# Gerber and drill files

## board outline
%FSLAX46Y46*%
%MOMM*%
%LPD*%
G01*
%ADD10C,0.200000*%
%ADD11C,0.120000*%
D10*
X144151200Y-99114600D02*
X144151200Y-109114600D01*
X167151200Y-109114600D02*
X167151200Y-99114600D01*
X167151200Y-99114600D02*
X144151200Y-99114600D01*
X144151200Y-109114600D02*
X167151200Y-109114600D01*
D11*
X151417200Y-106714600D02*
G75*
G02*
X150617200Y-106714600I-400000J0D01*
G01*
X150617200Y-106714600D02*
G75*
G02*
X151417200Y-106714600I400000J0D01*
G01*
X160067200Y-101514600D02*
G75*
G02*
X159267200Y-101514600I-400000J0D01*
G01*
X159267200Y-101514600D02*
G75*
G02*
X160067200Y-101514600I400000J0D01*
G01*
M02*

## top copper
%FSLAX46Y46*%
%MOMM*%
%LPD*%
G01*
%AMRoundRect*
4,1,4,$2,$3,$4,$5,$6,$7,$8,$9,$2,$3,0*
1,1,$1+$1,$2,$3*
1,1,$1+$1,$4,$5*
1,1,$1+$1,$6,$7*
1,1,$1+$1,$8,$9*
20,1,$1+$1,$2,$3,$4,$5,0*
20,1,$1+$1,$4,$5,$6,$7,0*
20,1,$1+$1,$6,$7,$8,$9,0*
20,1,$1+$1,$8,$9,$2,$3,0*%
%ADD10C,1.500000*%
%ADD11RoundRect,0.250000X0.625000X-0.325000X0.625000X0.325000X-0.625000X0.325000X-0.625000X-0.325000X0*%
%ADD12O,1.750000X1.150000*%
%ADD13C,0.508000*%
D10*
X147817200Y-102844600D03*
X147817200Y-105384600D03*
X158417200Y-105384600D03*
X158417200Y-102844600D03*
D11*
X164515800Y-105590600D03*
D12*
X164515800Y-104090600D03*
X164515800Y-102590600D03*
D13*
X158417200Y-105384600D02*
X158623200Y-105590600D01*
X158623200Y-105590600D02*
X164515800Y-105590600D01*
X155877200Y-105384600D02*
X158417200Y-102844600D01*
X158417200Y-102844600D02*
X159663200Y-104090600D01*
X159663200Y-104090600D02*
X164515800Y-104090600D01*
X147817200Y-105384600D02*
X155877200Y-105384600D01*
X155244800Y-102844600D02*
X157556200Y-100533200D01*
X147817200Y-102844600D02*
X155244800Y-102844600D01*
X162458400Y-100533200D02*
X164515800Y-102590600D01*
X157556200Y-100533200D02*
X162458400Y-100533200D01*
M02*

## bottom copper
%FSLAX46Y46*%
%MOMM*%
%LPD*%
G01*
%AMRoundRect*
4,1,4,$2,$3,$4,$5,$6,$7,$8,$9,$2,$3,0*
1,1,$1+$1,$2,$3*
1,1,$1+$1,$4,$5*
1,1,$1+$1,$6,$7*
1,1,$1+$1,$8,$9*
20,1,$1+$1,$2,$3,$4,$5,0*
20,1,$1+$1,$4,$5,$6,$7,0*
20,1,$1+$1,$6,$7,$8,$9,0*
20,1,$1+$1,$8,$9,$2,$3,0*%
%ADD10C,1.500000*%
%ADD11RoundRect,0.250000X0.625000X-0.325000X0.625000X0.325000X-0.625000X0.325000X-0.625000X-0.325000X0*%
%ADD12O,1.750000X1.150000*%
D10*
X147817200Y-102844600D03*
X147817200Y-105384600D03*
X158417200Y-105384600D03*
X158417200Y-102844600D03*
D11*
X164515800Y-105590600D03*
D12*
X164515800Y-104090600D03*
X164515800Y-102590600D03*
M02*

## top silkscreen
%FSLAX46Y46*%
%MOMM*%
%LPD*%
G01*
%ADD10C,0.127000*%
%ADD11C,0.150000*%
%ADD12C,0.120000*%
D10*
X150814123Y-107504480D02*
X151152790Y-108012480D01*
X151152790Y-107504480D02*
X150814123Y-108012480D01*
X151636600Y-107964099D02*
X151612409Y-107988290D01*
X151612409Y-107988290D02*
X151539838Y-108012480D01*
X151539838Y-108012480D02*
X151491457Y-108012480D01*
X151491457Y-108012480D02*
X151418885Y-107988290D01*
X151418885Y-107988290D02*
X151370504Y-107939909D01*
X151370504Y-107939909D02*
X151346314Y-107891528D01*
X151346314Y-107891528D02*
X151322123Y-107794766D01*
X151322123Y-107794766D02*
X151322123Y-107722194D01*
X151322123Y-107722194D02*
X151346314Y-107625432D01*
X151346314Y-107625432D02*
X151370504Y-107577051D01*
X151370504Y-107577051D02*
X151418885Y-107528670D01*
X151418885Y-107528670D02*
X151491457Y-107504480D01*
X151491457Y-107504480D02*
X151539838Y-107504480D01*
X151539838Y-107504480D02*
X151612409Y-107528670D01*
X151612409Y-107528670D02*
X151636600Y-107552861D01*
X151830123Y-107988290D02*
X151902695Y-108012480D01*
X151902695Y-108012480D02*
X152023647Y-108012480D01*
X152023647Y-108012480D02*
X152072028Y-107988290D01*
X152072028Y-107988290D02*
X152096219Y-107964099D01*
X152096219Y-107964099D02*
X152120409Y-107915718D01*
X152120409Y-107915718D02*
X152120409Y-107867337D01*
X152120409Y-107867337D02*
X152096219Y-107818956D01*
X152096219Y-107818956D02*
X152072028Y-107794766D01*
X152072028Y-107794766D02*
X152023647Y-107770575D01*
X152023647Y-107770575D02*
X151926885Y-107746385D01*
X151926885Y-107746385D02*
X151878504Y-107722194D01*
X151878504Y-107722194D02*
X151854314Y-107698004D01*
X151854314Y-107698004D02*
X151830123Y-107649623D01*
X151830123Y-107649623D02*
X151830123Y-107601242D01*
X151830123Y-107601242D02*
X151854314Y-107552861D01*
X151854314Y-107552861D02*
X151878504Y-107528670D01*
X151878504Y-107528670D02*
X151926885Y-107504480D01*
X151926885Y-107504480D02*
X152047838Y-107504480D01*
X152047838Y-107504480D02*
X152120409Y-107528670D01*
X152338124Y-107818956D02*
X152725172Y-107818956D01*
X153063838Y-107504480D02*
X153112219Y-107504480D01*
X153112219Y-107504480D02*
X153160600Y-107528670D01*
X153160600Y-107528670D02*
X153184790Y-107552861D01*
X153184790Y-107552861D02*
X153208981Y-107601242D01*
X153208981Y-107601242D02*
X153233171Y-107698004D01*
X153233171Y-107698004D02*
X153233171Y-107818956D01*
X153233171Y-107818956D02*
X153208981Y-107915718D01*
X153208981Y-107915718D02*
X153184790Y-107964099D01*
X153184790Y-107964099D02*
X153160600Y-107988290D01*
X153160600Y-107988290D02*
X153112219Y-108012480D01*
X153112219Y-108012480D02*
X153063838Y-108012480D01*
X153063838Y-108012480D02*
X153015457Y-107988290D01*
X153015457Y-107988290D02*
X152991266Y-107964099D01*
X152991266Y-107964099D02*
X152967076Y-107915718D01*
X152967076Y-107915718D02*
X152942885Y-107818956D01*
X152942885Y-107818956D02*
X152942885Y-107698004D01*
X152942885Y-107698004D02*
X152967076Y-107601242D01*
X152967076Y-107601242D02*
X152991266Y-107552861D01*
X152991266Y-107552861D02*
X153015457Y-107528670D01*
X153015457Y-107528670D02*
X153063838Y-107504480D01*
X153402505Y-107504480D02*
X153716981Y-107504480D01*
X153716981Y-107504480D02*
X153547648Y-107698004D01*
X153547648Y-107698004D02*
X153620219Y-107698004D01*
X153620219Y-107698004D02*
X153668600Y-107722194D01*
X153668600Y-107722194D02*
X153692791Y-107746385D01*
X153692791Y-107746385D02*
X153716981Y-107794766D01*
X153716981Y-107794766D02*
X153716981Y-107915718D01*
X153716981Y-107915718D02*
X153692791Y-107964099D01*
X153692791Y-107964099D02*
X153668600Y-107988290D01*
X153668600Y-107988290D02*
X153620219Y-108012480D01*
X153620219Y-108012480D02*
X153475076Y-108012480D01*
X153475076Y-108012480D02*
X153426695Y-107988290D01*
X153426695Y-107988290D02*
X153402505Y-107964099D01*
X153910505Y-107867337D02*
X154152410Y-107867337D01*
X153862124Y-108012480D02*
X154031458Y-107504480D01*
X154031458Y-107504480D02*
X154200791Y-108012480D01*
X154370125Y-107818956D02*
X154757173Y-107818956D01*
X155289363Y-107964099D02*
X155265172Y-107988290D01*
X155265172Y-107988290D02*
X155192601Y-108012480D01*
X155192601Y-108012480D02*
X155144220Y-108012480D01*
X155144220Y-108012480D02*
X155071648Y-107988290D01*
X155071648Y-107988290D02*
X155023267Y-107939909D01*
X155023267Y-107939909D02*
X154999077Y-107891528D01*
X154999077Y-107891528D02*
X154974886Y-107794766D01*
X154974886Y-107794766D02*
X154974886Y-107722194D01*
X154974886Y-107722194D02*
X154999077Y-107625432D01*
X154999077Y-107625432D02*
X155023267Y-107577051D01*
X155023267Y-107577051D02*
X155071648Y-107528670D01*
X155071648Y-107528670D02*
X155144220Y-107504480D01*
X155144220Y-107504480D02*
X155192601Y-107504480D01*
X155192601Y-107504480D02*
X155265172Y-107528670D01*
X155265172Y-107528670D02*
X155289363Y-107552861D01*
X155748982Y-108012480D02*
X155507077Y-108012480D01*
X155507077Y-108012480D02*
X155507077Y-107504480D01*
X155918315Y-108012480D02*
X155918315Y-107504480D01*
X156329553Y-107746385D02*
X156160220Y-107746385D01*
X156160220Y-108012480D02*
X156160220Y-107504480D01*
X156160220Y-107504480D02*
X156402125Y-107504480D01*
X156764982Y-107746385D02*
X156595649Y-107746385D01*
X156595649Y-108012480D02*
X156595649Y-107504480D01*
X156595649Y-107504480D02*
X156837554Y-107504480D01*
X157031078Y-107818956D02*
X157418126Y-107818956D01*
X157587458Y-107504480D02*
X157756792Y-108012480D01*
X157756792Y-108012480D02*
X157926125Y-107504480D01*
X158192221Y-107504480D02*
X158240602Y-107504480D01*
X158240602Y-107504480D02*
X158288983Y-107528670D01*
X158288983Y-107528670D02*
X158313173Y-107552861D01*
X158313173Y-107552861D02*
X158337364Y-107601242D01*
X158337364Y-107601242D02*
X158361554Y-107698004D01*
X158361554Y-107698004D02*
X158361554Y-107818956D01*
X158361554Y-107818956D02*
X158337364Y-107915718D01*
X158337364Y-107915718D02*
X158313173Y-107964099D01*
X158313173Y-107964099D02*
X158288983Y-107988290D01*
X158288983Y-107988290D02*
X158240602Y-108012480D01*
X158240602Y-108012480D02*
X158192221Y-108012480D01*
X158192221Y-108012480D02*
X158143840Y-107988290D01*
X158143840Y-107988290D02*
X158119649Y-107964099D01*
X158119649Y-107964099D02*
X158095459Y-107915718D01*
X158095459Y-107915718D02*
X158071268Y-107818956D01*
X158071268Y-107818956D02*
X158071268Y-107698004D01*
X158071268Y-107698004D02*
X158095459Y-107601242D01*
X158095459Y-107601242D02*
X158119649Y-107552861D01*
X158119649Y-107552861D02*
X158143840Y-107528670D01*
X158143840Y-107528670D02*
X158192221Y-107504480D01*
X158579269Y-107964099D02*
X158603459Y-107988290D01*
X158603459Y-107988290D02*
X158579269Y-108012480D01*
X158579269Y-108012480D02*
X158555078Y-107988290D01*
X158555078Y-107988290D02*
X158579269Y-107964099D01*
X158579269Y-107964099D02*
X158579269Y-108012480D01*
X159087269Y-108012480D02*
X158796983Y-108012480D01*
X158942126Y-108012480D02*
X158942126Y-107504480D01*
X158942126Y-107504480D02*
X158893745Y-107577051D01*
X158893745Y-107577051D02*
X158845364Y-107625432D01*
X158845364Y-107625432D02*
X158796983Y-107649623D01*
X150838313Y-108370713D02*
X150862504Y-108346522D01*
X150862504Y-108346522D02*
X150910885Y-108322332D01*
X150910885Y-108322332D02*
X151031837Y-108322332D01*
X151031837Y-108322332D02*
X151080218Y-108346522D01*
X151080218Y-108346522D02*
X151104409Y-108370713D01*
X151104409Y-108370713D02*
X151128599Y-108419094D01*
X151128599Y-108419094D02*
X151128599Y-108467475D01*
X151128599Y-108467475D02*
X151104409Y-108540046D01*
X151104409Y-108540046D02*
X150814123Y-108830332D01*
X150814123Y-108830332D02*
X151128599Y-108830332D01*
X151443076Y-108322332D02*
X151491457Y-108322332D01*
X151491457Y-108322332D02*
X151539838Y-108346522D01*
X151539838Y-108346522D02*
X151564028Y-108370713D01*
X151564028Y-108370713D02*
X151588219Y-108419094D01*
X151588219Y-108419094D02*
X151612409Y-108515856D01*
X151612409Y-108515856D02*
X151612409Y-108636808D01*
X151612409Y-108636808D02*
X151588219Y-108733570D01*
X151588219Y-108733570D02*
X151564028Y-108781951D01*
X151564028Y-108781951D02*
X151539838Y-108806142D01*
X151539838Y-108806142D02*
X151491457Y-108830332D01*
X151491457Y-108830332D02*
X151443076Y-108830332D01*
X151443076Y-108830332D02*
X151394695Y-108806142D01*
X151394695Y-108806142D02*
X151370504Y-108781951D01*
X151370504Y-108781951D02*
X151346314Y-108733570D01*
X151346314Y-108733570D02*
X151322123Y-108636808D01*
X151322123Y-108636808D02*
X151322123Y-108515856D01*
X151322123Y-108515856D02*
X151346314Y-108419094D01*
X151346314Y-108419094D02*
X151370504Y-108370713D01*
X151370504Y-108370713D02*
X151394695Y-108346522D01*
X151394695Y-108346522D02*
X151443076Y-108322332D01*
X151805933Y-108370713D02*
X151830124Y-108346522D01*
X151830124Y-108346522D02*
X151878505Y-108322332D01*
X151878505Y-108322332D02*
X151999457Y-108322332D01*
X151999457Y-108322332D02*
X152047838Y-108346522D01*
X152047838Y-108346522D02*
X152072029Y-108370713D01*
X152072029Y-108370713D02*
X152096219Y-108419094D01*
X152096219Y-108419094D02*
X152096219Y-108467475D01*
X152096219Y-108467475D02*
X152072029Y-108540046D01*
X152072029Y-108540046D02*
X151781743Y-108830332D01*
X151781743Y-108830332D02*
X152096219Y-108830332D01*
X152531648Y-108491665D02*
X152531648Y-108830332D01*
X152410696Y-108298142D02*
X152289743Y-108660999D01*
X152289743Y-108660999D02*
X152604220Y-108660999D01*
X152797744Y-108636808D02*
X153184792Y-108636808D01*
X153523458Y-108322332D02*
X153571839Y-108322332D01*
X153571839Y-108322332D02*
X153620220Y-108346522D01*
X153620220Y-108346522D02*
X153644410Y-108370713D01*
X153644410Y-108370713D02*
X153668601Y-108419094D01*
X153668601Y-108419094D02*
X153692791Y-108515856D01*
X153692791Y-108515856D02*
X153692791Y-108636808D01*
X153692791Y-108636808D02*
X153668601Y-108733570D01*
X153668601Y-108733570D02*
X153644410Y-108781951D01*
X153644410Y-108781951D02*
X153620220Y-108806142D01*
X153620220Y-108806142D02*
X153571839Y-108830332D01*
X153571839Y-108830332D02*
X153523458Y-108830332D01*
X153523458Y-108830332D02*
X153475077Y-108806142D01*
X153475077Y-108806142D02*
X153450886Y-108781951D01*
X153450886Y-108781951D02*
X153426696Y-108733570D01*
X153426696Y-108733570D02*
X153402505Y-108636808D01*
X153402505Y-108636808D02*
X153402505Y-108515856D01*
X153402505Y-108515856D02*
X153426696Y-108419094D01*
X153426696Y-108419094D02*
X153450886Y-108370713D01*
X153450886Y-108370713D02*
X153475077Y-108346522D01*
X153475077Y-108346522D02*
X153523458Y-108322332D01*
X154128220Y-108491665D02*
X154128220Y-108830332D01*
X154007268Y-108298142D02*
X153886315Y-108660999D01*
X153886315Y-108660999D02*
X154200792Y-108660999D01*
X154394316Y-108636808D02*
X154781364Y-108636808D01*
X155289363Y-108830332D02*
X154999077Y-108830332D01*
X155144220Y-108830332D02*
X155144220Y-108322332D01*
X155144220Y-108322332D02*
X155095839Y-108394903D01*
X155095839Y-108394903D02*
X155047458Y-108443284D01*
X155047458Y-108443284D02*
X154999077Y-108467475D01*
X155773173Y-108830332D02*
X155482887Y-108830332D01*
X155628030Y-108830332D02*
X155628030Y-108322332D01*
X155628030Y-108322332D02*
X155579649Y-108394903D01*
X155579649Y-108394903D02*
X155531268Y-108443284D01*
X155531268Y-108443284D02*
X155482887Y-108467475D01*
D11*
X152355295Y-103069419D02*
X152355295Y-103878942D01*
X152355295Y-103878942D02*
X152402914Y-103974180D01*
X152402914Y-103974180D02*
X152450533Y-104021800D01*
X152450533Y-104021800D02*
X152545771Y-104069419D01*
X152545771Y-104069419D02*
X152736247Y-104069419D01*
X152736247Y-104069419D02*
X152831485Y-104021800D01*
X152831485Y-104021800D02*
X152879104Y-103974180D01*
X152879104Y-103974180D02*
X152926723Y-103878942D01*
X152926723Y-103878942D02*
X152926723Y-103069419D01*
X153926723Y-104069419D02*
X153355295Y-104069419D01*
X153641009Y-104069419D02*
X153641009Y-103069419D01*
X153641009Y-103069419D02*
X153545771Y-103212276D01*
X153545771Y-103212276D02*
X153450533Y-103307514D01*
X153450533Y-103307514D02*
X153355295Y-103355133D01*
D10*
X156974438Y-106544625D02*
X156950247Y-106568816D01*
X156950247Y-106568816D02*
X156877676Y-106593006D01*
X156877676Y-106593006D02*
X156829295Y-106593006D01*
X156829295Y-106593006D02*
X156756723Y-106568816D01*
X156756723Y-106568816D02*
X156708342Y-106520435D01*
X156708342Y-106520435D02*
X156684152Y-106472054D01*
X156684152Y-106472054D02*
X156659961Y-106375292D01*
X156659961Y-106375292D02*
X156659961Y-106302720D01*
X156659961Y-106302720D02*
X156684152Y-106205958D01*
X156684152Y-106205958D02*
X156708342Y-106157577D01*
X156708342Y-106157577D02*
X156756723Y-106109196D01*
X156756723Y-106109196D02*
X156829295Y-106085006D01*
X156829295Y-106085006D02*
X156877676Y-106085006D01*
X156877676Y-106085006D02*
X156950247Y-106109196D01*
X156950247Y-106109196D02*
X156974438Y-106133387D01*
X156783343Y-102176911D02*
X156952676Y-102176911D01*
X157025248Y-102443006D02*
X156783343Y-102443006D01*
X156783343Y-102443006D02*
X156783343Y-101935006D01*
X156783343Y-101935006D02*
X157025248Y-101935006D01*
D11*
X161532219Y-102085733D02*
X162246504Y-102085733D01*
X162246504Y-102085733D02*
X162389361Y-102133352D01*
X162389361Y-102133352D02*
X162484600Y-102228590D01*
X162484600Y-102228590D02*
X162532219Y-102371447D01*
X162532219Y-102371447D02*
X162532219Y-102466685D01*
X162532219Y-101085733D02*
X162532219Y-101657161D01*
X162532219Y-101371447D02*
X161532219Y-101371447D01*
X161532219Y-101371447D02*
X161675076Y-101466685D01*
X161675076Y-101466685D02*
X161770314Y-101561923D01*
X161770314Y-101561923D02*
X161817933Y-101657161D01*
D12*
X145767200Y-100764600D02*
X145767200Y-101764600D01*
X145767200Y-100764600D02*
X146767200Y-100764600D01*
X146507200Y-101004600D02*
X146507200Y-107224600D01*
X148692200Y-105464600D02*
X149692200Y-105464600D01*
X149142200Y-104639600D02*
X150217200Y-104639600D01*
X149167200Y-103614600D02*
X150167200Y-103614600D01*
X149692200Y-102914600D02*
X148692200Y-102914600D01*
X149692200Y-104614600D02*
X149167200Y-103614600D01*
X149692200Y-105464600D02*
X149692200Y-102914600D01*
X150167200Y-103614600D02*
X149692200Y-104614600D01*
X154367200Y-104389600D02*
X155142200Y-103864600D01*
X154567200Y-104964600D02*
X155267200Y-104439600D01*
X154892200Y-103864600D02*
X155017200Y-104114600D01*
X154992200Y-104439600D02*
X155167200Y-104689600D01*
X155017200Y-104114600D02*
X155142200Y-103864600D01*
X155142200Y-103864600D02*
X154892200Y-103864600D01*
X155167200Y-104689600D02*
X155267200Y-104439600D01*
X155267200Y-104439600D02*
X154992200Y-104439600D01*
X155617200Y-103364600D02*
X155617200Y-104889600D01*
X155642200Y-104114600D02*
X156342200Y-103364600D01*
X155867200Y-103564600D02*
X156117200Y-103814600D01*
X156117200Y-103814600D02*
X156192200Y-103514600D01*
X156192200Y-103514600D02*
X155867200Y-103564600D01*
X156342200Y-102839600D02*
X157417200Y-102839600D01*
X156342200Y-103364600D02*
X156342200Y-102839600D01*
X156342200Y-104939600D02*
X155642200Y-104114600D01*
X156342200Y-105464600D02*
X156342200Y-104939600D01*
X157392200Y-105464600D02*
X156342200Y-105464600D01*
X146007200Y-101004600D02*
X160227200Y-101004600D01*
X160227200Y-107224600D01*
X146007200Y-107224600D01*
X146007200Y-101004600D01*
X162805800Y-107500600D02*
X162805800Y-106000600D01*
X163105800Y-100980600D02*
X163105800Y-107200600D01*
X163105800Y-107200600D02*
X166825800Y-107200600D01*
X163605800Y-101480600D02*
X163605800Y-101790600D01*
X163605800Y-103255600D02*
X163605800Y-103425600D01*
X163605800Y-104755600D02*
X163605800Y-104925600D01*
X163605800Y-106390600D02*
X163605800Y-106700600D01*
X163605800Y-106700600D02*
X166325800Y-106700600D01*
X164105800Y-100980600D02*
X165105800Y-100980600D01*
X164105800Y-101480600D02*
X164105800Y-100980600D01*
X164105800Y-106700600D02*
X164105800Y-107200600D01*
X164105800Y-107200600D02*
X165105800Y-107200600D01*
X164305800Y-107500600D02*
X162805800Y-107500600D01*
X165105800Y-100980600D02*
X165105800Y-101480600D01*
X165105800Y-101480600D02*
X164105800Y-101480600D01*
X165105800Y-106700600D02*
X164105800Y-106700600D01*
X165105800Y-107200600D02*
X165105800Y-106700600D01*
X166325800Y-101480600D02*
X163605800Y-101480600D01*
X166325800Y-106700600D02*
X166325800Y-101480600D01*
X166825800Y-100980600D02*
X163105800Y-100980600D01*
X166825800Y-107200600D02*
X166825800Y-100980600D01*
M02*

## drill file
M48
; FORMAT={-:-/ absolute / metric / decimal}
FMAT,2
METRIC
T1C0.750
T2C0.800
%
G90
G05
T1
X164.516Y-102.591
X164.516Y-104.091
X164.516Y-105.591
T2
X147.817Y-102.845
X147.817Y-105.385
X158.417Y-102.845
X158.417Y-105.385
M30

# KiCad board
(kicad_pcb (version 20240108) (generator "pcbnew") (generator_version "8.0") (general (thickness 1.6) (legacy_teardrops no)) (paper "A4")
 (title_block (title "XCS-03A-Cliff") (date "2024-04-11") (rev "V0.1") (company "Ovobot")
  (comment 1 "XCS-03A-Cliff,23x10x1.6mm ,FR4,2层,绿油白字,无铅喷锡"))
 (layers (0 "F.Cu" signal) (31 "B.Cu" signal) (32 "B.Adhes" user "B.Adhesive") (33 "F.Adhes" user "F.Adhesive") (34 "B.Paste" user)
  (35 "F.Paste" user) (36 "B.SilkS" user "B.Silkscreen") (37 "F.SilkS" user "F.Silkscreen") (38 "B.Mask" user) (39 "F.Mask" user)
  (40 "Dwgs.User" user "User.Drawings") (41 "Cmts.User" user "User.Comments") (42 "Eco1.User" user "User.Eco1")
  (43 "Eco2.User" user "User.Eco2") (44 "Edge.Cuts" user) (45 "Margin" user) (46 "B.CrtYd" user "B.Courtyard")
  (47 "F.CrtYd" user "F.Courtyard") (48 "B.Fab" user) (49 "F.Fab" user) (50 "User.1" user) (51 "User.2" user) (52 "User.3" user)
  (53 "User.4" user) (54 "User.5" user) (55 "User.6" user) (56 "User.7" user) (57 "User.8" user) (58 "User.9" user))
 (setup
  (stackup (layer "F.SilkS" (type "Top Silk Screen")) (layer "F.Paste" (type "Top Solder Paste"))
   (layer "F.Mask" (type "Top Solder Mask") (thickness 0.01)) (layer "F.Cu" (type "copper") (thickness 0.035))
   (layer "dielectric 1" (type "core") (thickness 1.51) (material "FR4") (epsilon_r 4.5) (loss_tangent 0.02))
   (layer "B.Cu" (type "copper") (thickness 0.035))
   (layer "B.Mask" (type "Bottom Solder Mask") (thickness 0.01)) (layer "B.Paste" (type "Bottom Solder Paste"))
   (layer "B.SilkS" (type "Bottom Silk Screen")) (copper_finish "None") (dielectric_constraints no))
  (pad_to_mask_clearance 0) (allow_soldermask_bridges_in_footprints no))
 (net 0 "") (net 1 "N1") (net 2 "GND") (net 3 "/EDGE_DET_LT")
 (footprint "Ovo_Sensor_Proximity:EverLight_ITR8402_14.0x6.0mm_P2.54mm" (layer "F.Cu") (at 153.1172 104.1146)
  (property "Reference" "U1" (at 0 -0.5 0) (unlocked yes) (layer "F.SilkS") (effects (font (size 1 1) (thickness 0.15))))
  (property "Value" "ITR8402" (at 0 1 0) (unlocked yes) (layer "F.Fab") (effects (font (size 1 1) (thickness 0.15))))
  (fp_line (start -7.35 -3.35) (end -7.35 -2.35) (stroke (width 0.12) (type solid)) (layer "F.SilkS"))
  (fp_line (start -7.35 -3.35) (end -6.35 -3.35) (stroke (width 0.12) (type solid)) (layer "F.SilkS"))
  (fp_line (start -6.61 -3.11) (end -6.61 3.11) (stroke (width 0.12) (type solid)) (layer "F.SilkS"))
  (fp_line (start -4.425 1.35) (end -3.425 1.35) (stroke (width 0.12) (type solid)) (layer "F.SilkS"))
  (fp_line (start -3.975 0.525) (end -2.9 0.525) (stroke (width 0.12) (type solid)) (layer "F.SilkS"))
  (fp_line (start -3.95 -0.5) (end -2.95 -0.5) (stroke (width 0.12) (type solid)) (layer "F.SilkS"))
  (fp_line (start -3.425 -1.2) (end -4.425 -1.2) (stroke (width 0.12) (type solid)) (layer "F.SilkS"))
  (fp_line (start -3.425 0.5) (end -3.95 -0.5) (stroke (width 0.12) (type solid)) (layer "F.SilkS"))
  (fp_line (start -3.425 1.35) (end -3.425 -1.2) (stroke (width 0.12) (type solid)) (layer "F.SilkS"))
  (fp_line (start -2.95 -0.5) (end -3.425 0.5) (stroke (width 0.12) (type solid)) (layer "F.SilkS"))
  (fp_line (start 1.25 0.275) (end 2.025 -0.25) (stroke (width 0.12) (type solid)) (layer "F.SilkS"))
  (fp_line (start 1.45 0.85) (end 2.15 0.325) (stroke (width 0.12) (type solid)) (layer "F.SilkS"))
  (fp_line (start 1.775 -0.25) (end 1.9 0) (stroke (width 0.12) (type solid)) (layer "F.SilkS"))
  (fp_line (start 1.875 0.325) (end 2.05 0.575) (stroke (width 0.12) (type solid)) (layer "F.SilkS"))
  (fp_line (start 1.9 0) (end 2.025 -0.25) (stroke (width 0.12) (type solid)) (layer "F.SilkS"))
  (fp_line (start 2.025 -0.25) (end 1.775 -0.25) (stroke (width 0.12) (type solid)) (layer "F.SilkS"))
  (fp_line (start 2.05 0.575) (end 2.15 0.325) (stroke (width 0.12) (type solid)) (layer "F.SilkS"))
  (fp_line (start 2.15 0.325) (end 1.875 0.325) (stroke (width 0.12) (type solid)) (layer "F.SilkS"))
  (fp_line (start 2.5 -0.75) (end 2.5 0.775) (stroke (width 0.12) (type solid)) (layer "F.SilkS"))
  (fp_line (start 2.525 0) (end 3.225 -0.75) (stroke (width 0.12) (type solid)) (layer "F.SilkS"))
  (fp_line (start 2.75 -0.55) (end 3 -0.3) (stroke (width 0.12) (type solid)) (layer "F.SilkS"))
  (fp_line (start 3 -0.3) (end 3.075 -0.6) (stroke (width 0.12) (type solid)) (layer "F.SilkS"))
  (fp_line (start 3.075 -0.6) (end 2.75 -0.55) (stroke (width 0.12) (type solid)) (layer "F.SilkS"))
  (fp_line (start 3.225 -1.275) (end 4.3 -1.275) (stroke (width 0.12) (type solid)) (layer "F.SilkS"))
  (fp_line (start 3.225 -0.75) (end 3.225 -1.275) (stroke (width 0.12) (type solid)) (layer "F.SilkS"))
  (fp_line (start 3.225 0.825) (end 2.525 0) (stroke (width 0.12) (type solid)) (layer "F.SilkS"))
  (fp_line (start 3.225 1.35) (end 3.225 0.825) (stroke (width 0.12) (type solid)) (layer "F.SilkS"))
  (fp_line (start 4.275 1.35) (end 3.225 1.35) (stroke (width 0.12) (type solid)) (layer "F.SilkS"))
  (fp_rect (start -7.11 -3.11) (end 7.11 3.11) (stroke (width 0.12) (type solid)) (fill none) (layer "F.SilkS"))
  (fp_circle (center -2.1 2.6) (end -1.7 2.6) (stroke (width 0.12) (type solid)) (fill none) (layer "Edge.Cuts"))
  (fp_circle (center 6.55 -2.6) (end 6.95 -2.6) (stroke (width 0.12) (type solid)) (fill none) (layer "Edge.Cuts"))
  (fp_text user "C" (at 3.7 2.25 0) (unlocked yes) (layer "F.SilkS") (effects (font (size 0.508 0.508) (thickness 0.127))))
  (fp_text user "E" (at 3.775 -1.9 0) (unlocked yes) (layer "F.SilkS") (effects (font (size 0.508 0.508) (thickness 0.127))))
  (pad "1" thru_hole circle (at -5.3 -1.27) (size 1.5 1.5) (drill 0.8) (layers "*.Cu" "*.Mask") (remove_unused_layers no) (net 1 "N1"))
  (pad "2" thru_hole circle (at -5.3 1.27) (size 1.5 1.5) (drill 0.8) (layers "*.Cu" "*.Mask") (remove_unused_layers no) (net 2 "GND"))
  (pad "3" thru_hole circle (at 5.3 1.27) (size 1.5 1.5) (drill 0.8) (layers "*.Cu" "*.Mask") (remove_unused_layers no)
   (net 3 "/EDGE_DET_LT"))
  (pad "4" thru_hole circle (at 5.3 -1.27) (size 1.5 1.5) (drill 0.8) (layers "*.Cu" "*.Mask") (remove_unused_layers no) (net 2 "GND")))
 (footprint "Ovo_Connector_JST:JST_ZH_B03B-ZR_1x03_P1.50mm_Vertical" (layer "F.Cu") (at 164.5158 105.5906 90)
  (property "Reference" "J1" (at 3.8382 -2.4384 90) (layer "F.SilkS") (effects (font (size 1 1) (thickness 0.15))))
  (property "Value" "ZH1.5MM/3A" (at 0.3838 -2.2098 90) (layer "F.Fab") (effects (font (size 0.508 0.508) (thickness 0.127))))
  (fp_line (start -1.91 -1.71) (end -0.41 -1.71) (stroke (width 0.12) (type solid)) (layer "F.SilkS"))
  (fp_line (start 4.61 -1.41) (end -1.61 -1.41) (stroke (width 0.12) (type solid)) (layer "F.SilkS"))
  (fp_line (start -1.61 -1.41) (end -1.61 2.31) (stroke (width 0.12) (type solid)) (layer "F.SilkS"))
  (fp_line (start 4.11 -0.91) (end 3.8 -0.91) (stroke (width 0.12) (type solid)) (layer "F.SilkS"))
  (fp_line (start 2.335 -0.91) (end 2.165 -0.91) (stroke (width 0.12) (type solid)) (layer "F.SilkS"))
  (fp_line (start 0.835 -0.91) (end 0.665 -0.91) (stroke (width 0.12) (type solid)) (layer "F.SilkS"))
  (fp_line (start -0.8 -0.91) (end -1.11 -0.91) (stroke (width 0.12) (type solid)) (layer "F.SilkS"))
  (fp_line (start -1.11 -0.91) (end -1.11 1.81) (stroke (width 0.12) (type solid)) (layer "F.SilkS"))
  (fp_line (start 4.61 -0.41) (end 4.61 0.59) (stroke (width 0.12) (type solid)) (layer "F.SilkS"))
  (fp_line (start 4.11 -0.41) (end 4.61 -0.41) (stroke (width 0.12) (type solid)) (layer "F.SilkS"))
  (fp_line (start -1.11 -0.41) (end -1.61 -0.41) (stroke (width 0.12) (type solid)) (layer "F.SilkS"))
  (fp_line (start -1.61 -0.41) (end -1.61 0.59) (stroke (width 0.12) (type solid)) (layer "F.SilkS"))
  (fp_line (start -1.91 -0.21) (end -1.91 -1.71) (stroke (width 0.12) (type solid)) (layer "F.SilkS"))
  (fp_line (start 4.61 0.59) (end 4.11 0.59) (stroke (width 0.12) (type solid)) (layer "F.SilkS"))
  (fp_line (start 4.11 0.59) (end 4.11 -0.41) (stroke (width 0.12) (type solid)) (layer "F.SilkS"))
  (fp_line (start -1.11 0.59) (end -1.11 -0.41) (stroke (width 0.12) (type solid)) (layer "F.SilkS"))
  (fp_line (start -1.61 0.59) (end -1.11 0.59) (stroke (width 0.12) (type solid)) (layer "F.SilkS"))
  (fp_line (start 4.11 1.81) (end 4.11 -0.91) (stroke (width 0.12) (type solid)) (layer "F.SilkS"))
  (fp_line (start -1.11 1.81) (end 4.11 1.81) (stroke (width 0.12) (type solid)) (layer "F.SilkS"))
  (fp_line (start 4.61 2.31) (end 4.61 -1.41) (stroke (width 0.12) (type solid)) (layer "F.SilkS"))
  (fp_line (start -1.61 2.31) (end 4.61 2.31) (stroke (width 0.12) (type solid)) (layer "F.SilkS"))
  (pad "1" thru_hole roundrect (at 0 0 90) (size 1.15 1.75) (drill 0.75) (layers "*.Cu" "*.Mask") (remove_unused_layers no)
   (roundrect_rratio 0.2173913043) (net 3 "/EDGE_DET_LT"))
  (pad "2" thru_hole oval (at 1.5 0 90) (size 1.15 1.75) (drill 0.75) (layers "*.Cu" "*.Mask") (remove_unused_layers no) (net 2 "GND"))
  (pad "3" thru_hole oval (at 3 0 90) (size 1.15 1.75) (drill 0.75) (layers "*.Cu" "*.Mask") (remove_unused_layers no) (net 1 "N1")))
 (gr_line (start 144.1512 99.1146) (end 144.1512 109.1146) (stroke (width 0.2) (type solid)) (layer "Edge.Cuts"))
 (gr_line (start 167.1512 109.1146) (end 167.1512 99.1146) (stroke (width 0.2) (type solid)) (layer "Edge.Cuts"))
 (gr_line (start 167.1512 99.1146) (end 144.1512 99.1146) (stroke (width 0.2) (type solid)) (layer "Edge.Cuts"))
 (gr_line (start 144.1512 109.1146) (end 167.1512 109.1146) (stroke (width 0.2) (type solid)) (layer "Edge.Cuts"))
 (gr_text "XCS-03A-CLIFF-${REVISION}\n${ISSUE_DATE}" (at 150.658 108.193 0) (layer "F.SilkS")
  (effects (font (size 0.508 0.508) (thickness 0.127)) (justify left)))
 (segment (start 158.4172 105.3846) (end 158.6232 105.5906) (width 0.508) (layer "F.Cu") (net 3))
 (segment (start 158.6232 105.5906) (end 164.5158 105.5906) (width 0.508) (layer "F.Cu") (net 3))
 (segment (start 155.8772 105.3846) (end 158.4172 102.8446) (width 0.508) (layer "F.Cu") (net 2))
 (segment (start 158.4172 102.8446) (end 159.6632 104.0906) (width 0.508) (layer "F.Cu") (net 2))
 (segment (start 159.6632 104.0906) (end 164.5158 104.0906) (width 0.508) (layer "F.Cu") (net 2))
 (segment (start 147.8172 105.3846) (end 155.8772 105.3846) (width 0.508) (layer "F.Cu") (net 2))
 (segment (start 155.2448 102.8446) (end 157.5562 100.5332) (width 0.508) (layer "F.Cu") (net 1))
 (segment (start 147.8172 102.8446) (end 155.2448 102.8446) (width 0.508) (layer "F.Cu") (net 1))
 (segment (start 162.4584 100.5332) (end 164.5158 102.5906) (width 0.508) (layer "F.Cu") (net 1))
 (segment (start 157.5562 100.5332) (end 162.4584 100.5332) (width 0.508) (layer "F.Cu") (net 1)))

